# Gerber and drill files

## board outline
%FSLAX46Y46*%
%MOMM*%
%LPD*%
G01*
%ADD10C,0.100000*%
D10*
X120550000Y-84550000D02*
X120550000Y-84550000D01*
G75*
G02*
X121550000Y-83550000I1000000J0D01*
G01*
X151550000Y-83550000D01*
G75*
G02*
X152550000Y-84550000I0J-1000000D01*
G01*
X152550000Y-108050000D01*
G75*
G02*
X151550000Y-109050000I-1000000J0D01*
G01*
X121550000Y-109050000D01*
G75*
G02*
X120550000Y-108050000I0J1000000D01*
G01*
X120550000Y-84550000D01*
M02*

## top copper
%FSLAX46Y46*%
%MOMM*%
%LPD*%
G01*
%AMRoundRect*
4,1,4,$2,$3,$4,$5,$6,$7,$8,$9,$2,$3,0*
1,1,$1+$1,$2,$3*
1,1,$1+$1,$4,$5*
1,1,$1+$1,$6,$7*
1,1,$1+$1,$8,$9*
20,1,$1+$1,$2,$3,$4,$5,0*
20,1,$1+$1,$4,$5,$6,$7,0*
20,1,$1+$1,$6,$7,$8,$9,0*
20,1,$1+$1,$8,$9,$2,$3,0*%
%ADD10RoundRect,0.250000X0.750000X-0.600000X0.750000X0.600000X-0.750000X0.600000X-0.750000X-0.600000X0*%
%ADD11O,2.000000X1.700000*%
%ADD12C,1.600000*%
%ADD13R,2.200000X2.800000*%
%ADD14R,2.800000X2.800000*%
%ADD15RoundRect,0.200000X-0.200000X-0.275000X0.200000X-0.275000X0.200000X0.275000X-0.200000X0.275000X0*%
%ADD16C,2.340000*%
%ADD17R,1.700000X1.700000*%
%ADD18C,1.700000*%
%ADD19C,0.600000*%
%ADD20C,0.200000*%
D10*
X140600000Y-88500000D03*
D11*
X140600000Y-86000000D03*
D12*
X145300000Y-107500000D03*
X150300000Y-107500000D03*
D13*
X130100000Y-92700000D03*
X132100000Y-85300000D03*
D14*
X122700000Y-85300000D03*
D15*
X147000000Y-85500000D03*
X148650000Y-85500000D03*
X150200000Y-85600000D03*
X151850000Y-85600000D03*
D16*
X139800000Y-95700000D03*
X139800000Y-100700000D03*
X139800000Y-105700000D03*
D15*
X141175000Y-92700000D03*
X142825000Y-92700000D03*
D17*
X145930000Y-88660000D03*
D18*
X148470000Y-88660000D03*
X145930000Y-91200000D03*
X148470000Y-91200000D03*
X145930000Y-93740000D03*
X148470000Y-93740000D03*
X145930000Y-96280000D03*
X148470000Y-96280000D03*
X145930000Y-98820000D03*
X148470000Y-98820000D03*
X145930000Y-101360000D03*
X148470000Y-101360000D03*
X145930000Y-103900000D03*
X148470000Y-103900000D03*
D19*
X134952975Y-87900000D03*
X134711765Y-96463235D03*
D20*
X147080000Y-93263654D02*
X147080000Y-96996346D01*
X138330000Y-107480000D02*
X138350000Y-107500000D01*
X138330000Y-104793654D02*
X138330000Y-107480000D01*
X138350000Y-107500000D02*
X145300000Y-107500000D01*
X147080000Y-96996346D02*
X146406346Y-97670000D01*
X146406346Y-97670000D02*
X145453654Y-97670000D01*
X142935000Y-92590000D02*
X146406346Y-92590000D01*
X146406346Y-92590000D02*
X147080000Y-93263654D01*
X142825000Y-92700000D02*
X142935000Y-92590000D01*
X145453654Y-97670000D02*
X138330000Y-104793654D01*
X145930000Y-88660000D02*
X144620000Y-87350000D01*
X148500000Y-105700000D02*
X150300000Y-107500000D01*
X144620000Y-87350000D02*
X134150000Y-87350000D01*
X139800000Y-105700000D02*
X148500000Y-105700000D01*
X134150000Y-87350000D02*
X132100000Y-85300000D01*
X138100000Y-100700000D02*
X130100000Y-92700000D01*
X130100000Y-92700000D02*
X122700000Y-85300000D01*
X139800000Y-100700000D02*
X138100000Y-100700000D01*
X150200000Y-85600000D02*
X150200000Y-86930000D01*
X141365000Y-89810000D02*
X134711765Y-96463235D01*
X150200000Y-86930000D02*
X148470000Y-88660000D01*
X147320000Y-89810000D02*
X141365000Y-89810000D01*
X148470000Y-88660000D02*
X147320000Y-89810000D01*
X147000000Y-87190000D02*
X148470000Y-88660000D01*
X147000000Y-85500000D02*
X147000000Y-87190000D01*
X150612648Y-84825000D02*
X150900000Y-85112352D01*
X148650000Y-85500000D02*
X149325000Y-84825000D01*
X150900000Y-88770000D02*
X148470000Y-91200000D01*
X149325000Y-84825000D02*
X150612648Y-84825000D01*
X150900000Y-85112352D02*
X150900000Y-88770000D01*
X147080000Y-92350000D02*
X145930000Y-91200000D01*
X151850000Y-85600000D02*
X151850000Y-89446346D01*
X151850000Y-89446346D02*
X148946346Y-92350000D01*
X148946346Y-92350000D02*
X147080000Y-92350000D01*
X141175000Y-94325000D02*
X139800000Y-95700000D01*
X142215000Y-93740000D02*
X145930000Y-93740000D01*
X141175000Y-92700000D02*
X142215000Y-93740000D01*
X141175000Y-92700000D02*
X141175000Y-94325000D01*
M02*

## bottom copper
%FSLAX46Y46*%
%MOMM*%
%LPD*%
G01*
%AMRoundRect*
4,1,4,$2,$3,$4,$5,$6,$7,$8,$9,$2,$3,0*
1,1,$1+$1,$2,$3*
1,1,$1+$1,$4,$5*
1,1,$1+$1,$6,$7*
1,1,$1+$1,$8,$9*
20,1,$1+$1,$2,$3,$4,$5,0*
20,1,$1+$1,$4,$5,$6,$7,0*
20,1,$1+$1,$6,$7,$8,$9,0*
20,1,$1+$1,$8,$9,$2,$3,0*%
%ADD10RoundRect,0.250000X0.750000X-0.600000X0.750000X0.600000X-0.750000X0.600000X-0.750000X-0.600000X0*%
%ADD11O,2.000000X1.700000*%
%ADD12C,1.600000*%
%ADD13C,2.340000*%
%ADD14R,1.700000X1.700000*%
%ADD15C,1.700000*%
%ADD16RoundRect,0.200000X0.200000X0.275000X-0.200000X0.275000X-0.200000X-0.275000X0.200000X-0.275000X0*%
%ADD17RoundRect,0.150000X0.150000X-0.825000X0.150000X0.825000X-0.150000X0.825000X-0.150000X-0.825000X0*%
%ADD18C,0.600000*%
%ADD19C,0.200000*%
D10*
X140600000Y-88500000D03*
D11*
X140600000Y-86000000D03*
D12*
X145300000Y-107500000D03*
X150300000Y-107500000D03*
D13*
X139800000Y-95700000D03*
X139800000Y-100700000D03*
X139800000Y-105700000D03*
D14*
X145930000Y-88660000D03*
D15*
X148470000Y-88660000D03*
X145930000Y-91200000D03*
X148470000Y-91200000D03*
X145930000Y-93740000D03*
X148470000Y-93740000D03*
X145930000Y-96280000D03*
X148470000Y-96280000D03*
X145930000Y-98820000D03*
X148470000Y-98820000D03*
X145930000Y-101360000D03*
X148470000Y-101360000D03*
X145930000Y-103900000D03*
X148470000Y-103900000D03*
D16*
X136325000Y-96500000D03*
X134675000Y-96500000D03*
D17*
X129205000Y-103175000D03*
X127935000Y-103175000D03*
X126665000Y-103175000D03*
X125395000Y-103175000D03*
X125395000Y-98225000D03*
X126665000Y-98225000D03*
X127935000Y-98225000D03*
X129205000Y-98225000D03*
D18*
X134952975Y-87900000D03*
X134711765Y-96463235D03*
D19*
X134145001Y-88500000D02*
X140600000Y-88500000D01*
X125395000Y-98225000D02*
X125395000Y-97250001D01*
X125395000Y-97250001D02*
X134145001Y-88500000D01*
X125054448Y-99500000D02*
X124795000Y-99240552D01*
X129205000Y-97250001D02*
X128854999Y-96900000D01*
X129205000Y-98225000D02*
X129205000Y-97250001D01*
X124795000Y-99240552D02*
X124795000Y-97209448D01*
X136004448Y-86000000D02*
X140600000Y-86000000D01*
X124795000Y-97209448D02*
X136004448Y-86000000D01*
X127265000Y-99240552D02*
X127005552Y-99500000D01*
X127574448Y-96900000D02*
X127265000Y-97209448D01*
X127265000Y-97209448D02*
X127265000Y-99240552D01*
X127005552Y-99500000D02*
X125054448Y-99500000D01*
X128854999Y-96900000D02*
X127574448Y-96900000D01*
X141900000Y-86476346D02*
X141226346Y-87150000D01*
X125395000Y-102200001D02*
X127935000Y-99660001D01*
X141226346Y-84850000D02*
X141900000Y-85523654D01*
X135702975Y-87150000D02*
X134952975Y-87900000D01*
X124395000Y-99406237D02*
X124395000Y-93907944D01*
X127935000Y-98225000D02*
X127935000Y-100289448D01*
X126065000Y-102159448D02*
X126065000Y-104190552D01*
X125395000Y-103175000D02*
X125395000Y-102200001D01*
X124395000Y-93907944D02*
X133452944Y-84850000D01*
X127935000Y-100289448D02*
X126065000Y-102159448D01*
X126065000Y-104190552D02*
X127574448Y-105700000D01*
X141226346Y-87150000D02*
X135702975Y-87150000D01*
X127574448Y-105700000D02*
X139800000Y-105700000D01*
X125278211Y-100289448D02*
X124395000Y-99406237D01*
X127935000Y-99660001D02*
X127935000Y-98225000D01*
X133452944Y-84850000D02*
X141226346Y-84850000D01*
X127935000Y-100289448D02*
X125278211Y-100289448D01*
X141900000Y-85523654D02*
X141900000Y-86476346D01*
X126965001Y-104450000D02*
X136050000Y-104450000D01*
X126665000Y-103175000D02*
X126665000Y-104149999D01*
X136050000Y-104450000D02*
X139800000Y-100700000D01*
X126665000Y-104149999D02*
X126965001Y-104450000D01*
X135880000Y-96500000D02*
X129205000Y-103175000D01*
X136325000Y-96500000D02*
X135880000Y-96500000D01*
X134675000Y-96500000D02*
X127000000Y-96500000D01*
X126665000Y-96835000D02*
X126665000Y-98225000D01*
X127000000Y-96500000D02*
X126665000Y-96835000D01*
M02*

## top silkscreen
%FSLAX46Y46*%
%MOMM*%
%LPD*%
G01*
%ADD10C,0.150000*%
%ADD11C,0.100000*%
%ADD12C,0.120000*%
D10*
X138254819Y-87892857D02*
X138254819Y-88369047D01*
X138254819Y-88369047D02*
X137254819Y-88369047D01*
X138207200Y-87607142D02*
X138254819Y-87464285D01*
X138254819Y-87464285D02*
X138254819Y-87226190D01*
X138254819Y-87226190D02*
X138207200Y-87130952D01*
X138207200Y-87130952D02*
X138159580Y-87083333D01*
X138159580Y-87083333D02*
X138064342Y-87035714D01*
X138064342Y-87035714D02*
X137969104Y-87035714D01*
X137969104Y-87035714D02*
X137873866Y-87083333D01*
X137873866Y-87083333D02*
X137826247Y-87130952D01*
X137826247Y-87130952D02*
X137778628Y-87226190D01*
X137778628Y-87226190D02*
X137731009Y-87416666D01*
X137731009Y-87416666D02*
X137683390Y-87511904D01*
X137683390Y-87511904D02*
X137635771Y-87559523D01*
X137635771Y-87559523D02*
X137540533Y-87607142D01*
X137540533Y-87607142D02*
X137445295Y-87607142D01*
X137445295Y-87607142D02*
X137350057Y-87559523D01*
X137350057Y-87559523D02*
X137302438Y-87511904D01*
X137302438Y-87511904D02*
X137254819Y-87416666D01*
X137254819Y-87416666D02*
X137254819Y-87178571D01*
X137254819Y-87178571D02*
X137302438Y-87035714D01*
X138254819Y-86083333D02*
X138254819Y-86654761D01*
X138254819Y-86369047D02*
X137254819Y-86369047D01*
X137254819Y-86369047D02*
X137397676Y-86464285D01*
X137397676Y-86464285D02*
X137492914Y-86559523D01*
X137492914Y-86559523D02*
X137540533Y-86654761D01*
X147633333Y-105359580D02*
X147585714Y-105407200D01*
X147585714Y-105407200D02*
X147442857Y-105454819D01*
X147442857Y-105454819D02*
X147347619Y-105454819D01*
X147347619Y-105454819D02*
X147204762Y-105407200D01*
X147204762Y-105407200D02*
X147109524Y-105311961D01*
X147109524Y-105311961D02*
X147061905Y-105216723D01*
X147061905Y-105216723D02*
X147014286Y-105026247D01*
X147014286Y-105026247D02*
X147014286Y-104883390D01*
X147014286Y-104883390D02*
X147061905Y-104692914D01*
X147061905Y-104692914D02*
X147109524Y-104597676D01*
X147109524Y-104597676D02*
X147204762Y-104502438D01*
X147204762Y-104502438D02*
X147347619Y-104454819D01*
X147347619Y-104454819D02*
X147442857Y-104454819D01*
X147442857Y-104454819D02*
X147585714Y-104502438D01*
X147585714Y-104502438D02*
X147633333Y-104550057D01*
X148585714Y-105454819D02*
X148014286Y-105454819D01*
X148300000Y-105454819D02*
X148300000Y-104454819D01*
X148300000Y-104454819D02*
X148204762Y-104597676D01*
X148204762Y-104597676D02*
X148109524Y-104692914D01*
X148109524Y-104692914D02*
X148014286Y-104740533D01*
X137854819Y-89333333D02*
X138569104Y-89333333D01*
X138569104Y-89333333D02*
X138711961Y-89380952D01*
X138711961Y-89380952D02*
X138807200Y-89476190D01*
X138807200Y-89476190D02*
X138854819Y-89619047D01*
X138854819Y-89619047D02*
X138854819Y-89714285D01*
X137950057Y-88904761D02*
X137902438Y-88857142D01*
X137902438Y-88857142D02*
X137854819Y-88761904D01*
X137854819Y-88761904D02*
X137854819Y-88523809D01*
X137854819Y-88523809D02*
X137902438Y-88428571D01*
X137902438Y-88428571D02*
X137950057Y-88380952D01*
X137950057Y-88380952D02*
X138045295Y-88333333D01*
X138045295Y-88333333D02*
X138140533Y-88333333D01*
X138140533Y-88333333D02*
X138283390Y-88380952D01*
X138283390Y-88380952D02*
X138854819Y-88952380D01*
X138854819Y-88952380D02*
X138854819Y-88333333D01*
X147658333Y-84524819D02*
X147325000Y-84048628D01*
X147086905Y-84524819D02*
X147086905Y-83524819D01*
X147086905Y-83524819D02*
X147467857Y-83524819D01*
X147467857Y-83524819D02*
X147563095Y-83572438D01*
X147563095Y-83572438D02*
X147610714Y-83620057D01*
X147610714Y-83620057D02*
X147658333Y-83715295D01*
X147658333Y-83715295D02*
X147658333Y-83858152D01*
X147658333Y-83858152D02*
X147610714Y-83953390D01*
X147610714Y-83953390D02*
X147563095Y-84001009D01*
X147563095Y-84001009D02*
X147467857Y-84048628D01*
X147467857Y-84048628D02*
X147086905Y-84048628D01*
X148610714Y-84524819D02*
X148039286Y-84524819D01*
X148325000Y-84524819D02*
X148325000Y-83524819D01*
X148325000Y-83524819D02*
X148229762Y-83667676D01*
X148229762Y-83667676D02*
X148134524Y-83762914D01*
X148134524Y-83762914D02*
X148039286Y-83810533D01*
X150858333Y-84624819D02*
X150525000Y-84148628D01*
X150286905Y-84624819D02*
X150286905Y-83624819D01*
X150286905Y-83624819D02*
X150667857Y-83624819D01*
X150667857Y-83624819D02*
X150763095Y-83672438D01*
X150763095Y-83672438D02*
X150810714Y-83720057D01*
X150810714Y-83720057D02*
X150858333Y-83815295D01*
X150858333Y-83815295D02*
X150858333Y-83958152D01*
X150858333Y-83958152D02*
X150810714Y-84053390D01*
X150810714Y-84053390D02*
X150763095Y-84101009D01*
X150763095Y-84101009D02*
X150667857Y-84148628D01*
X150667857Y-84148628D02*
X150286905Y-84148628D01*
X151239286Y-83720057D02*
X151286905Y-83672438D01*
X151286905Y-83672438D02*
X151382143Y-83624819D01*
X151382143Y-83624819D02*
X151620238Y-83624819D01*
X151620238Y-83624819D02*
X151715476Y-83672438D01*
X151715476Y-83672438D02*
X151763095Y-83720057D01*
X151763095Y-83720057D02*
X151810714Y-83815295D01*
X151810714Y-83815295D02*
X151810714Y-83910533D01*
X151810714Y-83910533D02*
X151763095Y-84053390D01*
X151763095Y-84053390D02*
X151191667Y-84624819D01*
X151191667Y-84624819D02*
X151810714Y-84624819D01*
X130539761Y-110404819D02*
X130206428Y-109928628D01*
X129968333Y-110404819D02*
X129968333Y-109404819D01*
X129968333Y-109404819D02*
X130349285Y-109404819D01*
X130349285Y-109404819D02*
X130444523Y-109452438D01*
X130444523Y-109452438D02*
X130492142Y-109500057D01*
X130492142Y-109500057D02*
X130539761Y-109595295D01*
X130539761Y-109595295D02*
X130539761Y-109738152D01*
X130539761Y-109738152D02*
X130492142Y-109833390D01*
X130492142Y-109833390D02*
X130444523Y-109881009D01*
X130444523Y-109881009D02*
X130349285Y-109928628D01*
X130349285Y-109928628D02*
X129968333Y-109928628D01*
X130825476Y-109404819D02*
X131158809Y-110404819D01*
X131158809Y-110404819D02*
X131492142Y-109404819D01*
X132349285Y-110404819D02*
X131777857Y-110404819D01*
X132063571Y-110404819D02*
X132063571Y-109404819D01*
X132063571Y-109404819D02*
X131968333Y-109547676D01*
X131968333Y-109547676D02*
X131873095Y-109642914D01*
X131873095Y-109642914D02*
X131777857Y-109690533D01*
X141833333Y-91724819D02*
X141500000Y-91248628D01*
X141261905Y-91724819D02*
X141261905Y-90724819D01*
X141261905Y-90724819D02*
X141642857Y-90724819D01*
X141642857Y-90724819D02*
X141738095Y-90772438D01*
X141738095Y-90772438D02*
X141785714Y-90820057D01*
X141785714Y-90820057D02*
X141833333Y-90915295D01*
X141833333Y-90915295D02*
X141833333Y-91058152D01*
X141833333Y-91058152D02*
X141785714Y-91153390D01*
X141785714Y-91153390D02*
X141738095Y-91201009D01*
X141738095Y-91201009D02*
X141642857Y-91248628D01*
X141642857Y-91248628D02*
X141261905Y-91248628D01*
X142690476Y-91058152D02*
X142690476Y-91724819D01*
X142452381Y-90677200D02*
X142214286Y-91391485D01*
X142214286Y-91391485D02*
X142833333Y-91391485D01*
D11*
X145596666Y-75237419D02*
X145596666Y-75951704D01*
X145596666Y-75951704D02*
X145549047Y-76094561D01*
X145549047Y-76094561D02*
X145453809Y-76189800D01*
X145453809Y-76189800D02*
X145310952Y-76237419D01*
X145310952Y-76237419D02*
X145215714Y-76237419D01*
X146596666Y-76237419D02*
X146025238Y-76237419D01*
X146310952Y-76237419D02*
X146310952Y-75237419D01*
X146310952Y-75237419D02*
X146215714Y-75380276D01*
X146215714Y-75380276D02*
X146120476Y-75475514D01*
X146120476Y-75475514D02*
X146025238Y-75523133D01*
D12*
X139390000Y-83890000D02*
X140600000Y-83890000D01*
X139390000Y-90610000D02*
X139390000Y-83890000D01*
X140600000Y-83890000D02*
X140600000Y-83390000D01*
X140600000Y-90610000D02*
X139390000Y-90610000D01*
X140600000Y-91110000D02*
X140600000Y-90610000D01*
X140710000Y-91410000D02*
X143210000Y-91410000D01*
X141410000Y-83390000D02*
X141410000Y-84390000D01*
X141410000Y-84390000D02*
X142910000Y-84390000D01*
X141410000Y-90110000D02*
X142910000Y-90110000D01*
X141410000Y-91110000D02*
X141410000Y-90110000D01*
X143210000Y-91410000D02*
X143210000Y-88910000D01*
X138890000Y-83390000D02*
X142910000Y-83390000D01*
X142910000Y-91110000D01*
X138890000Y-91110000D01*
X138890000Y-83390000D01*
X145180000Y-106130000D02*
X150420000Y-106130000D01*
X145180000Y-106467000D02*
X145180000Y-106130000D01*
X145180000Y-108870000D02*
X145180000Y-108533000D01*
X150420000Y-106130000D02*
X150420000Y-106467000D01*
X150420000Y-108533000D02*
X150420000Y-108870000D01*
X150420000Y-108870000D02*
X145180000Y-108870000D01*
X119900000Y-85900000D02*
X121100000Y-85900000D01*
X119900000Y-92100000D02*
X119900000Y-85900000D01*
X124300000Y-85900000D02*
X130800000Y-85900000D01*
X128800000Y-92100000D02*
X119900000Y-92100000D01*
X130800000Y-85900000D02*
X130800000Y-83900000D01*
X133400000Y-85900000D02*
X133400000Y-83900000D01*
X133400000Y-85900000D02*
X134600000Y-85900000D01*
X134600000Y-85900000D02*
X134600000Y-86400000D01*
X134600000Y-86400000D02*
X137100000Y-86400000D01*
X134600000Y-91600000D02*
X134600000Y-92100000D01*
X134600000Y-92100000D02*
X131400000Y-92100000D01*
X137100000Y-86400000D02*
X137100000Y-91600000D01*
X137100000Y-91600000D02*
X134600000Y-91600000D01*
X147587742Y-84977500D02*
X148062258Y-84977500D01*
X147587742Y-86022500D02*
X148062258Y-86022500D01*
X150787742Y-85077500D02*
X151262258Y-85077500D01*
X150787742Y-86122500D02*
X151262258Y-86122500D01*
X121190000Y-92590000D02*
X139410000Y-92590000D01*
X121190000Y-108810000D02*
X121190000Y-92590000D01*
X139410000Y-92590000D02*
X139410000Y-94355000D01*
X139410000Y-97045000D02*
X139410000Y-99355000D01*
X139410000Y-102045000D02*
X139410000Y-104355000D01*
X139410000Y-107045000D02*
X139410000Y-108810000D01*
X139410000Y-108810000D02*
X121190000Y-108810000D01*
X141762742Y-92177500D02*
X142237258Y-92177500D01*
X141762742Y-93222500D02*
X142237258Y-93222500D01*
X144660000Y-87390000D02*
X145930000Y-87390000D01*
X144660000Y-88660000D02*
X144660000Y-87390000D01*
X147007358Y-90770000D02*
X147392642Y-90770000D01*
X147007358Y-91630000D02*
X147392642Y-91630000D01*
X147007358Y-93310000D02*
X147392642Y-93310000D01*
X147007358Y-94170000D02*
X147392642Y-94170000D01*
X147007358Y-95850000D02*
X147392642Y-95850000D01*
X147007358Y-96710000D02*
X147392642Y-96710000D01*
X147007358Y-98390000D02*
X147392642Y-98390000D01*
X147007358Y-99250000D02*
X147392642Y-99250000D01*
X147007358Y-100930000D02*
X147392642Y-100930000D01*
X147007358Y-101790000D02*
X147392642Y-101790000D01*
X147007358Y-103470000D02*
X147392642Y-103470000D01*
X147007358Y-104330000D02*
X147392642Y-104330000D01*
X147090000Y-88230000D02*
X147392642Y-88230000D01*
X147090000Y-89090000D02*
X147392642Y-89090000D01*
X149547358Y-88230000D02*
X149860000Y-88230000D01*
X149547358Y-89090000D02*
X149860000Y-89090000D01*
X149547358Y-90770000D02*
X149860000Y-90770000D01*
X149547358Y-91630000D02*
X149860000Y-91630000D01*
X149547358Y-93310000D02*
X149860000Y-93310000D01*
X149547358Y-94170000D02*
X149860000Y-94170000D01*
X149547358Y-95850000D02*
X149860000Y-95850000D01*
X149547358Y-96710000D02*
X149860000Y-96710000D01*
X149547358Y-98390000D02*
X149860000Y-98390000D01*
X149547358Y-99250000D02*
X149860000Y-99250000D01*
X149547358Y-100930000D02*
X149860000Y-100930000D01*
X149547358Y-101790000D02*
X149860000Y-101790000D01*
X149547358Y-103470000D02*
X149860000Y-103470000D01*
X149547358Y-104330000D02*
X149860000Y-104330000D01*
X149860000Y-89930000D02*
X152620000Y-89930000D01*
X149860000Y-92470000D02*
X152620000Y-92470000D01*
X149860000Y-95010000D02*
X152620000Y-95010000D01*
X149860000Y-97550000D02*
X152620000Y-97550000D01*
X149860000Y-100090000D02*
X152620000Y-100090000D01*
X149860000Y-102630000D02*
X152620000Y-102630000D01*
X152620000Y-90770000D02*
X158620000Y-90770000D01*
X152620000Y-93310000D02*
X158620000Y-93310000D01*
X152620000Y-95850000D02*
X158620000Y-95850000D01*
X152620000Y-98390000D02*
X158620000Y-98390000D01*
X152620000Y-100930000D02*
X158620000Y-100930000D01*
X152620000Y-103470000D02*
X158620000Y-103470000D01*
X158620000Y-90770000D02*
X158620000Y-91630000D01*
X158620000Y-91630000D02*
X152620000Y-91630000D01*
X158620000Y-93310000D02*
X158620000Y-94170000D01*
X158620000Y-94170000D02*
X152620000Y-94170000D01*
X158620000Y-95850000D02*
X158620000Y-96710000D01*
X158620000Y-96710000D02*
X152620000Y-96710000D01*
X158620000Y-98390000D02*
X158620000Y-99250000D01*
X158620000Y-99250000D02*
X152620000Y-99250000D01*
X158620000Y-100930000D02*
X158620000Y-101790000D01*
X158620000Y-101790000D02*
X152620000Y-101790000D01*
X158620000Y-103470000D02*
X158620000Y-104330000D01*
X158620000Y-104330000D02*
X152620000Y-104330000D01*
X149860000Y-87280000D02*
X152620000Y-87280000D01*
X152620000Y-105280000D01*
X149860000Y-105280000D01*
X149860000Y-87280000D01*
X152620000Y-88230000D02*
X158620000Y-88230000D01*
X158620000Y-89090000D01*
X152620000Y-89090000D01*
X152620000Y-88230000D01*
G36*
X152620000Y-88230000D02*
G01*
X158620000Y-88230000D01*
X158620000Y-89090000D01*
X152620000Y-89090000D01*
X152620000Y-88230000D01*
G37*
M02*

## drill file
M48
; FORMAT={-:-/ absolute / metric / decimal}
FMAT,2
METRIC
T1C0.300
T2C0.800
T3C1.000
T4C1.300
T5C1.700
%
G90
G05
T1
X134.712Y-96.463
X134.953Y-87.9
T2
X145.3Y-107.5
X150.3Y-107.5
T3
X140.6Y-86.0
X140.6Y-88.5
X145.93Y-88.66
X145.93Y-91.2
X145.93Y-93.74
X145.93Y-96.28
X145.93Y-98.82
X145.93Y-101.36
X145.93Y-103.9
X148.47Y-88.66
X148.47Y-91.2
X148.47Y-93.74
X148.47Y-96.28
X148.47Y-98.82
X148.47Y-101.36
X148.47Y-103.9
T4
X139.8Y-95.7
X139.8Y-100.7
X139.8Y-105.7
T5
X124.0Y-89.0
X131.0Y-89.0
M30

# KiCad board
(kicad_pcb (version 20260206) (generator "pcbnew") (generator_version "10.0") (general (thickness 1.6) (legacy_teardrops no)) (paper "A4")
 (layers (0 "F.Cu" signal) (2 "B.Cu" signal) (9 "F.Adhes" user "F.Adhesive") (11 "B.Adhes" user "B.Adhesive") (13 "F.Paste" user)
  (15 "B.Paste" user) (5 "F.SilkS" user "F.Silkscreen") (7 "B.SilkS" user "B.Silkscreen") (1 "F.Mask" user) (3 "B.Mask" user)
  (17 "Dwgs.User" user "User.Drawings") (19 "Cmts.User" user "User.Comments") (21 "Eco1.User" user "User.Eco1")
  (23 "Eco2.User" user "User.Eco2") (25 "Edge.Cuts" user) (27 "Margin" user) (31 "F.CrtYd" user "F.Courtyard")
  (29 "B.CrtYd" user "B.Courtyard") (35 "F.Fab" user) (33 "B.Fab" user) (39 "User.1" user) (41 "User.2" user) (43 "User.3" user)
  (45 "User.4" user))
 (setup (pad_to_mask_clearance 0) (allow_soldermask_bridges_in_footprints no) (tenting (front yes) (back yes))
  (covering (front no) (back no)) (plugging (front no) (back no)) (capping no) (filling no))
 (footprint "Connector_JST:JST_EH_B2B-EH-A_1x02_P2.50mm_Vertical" (layer "F.Cu") (at 140.6 88.5 90)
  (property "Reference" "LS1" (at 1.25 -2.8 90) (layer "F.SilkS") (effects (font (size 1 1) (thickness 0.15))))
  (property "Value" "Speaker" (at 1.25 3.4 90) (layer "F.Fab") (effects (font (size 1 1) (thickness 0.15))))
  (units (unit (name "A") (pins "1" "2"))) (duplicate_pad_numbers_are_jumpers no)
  (fp_line (start 4.61 -1.21) (end 4.61 0) (stroke (width 0.12) (type solid)) (layer "F.SilkS"))
  (fp_line (start -2.11 -1.21) (end 4.61 -1.21) (stroke (width 0.12) (type solid)) (layer "F.SilkS"))
  (fp_line (start 4.61 0) (end 5.11 0) (stroke (width 0.12) (type solid)) (layer "F.SilkS"))
  (fp_line (start -2.11 0) (end -2.11 -1.21) (stroke (width 0.12) (type solid)) (layer "F.SilkS"))
  (fp_line (start -2.61 0) (end -2.11 0) (stroke (width 0.12) (type solid)) (layer "F.SilkS"))
  (fp_line (start -2.91 0.11) (end -2.91 2.61) (stroke (width 0.12) (type solid)) (layer "F.SilkS"))
  (fp_line (start 5.11 0.81) (end 4.11 0.81) (stroke (width 0.12) (type solid)) (layer "F.SilkS"))
  (fp_line (start 4.11 0.81) (end 4.11 2.31) (stroke (width 0.12) (type solid)) (layer "F.SilkS"))
  (fp_line (start -1.61 0.81) (end -1.61 2.31) (stroke (width 0.12) (type solid)) (layer "F.SilkS"))
  (fp_line (start -2.61 0.81) (end -1.61 0.81) (stroke (width 0.12) (type solid)) (layer "F.SilkS"))
  (fp_line (start -2.91 2.61) (end -0.41 2.61) (stroke (width 0.12) (type solid)) (layer "F.SilkS"))
  (fp_rect (start -2.61 -1.71) (end 5.11 2.31) (stroke (width 0.12) (type solid)) (fill no) (layer "F.SilkS"))
  (pad "1" thru_hole roundrect (at 0 0 90) (size 1.7 2) (drill 1) (layers "*.Cu" "*.Mask") (remove_unused_layers no)
   (roundrect_rratio 0.147059) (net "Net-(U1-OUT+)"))
  (pad "2" thru_hole oval (at 2.5 0 90) (size 1.7 2) (drill 1) (layers "*.Cu" "*.Mask") (remove_unused_layers no) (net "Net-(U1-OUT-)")))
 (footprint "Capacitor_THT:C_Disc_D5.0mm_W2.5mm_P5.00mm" (layer "F.Cu") (at 145.3 107.5)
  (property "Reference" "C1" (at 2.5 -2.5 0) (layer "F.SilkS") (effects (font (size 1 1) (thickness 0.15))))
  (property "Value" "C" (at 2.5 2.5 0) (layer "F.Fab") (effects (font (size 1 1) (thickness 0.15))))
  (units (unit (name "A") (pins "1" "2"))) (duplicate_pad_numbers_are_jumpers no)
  (fp_line (start -0.12 -1.37) (end 5.12 -1.37) (stroke (width 0.12) (type solid)) (layer "F.SilkS"))
  (fp_line (start -0.12 -1.033) (end -0.12 -1.37) (stroke (width 0.12) (type solid)) (layer "F.SilkS"))
  (fp_line (start -0.12 1.37) (end -0.12 1.033) (stroke (width 0.12) (type solid)) (layer "F.SilkS"))
  (fp_line (start 5.12 -1.37) (end 5.12 -1.033) (stroke (width 0.12) (type solid)) (layer "F.SilkS"))
  (fp_line (start 5.12 1.033) (end 5.12 1.37) (stroke (width 0.12) (type solid)) (layer "F.SilkS"))
  (fp_line (start 5.12 1.37) (end -0.12 1.37) (stroke (width 0.12) (type solid)) (layer "F.SilkS"))
  (pad "1" thru_hole circle (at 0 0) (size 1.6 1.6) (drill 0.8) (layers "*.Cu" "*.Mask") (remove_unused_layers no) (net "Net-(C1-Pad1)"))
  (pad "2" thru_hole circle (at 5 0) (size 1.6 1.6) (drill 0.8) (layers "*.Cu" "*.Mask") (remove_unused_layers no) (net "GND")))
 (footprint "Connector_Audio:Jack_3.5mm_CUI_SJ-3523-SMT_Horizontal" (layer "F.Cu") (at 128.5 89 -90)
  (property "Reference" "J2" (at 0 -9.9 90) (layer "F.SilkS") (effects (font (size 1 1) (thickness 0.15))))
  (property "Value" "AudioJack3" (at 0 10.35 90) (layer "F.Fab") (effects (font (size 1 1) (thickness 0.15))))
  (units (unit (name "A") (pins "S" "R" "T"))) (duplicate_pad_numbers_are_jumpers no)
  (fp_line (start -3.1 8.6) (end -3.1 7.4) (stroke (width 0.12) (type solid)) (layer "F.SilkS"))
  (fp_line (start 3.1 8.6) (end -3.1 8.6) (stroke (width 0.12) (type solid)) (layer "F.SilkS"))
  (fp_line (start -3.1 4.2) (end -3.1 -2.3) (stroke (width 0.12) (type solid)) (layer "F.SilkS"))
  (fp_line (start 3.1 -0.3) (end 3.1 8.6) (stroke (width 0.12) (type solid)) (layer "F.SilkS"))
  (fp_line (start -3.1 -2.3) (end -5.1 -2.3) (stroke (width 0.12) (type solid)) (layer "F.SilkS"))
  (fp_line (start -3.1 -4.9) (end -5.1 -4.9) (stroke (width 0.12) (type solid)) (layer "F.SilkS"))
  (fp_line (start -3.1 -4.9) (end -3.1 -6.1) (stroke (width 0.12) (type solid)) (layer "F.SilkS"))
  (fp_line (start -3.1 -6.1) (end -2.6 -6.1) (stroke (width 0.12) (type solid)) (layer "F.SilkS"))
  (fp_line (start -2.6 -6.1) (end -2.6 -8.6) (stroke (width 0.12) (type solid)) (layer "F.SilkS"))
  (fp_line (start 2.6 -6.1) (end 3.1 -6.1) (stroke (width 0.12) (type solid)) (layer "F.SilkS"))
  (fp_line (start 3.1 -6.1) (end 3.1 -2.9) (stroke (width 0.12) (type solid)) (layer "F.SilkS"))
  (fp_line (start -2.6 -8.6) (end 2.6 -8.6) (stroke (width 0.12) (type solid)) (layer "F.SilkS"))
  (fp_line (start 2.6 -8.6) (end 2.6 -6.1) (stroke (width 0.12) (type solid)) (layer "F.SilkS"))
  (pad "" np_thru_hole circle (at 0 -2.5 270) (size 1.7 1.7) (drill 1.7) (layers "*.Cu" "*.Mask"))
  (pad "" np_thru_hole circle (at 0 4.5 270) (size 1.7 1.7) (drill 1.7) (layers "*.Cu" "*.Mask"))
  (pad "R" smd rect (at 3.7 -1.6 270) (size 2.8 2.2) (layers "F.Cu" "F.Mask" "F.Paste") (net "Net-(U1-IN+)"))
  (pad "S" smd rect (at -3.7 -3.6 270) (size 2.8 2.2) (layers "F.Cu" "F.Mask" "F.Paste") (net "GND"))
  (pad "T" smd rect (at -3.7 5.8 270) (size 2.8 2.8) (layers "F.Cu" "F.Mask" "F.Paste") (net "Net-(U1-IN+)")))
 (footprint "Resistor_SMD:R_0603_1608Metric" (layer "F.Cu") (at 147.825 85.5)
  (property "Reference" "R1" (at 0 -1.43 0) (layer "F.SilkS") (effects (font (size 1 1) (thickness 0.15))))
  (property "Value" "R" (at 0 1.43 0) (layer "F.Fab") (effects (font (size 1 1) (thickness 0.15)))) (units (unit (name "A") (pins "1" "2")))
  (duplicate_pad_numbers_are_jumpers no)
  (fp_line (start -0.237258 -0.5225) (end 0.237258 -0.5225) (stroke (width 0.12) (type solid)) (layer "F.SilkS"))
  (fp_line (start -0.237258 0.5225) (end 0.237258 0.5225) (stroke (width 0.12) (type solid)) (layer "F.SilkS"))
  (pad "1" smd roundrect (at -0.825 0) (size 0.8 0.95) (layers "F.Cu" "F.Mask" "F.Paste") (roundrect_rratio 0.25) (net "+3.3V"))
  (pad "2" smd roundrect (at 0.825 0) (size 0.8 0.95) (layers "F.Cu" "F.Mask" "F.Paste") (roundrect_rratio 0.25) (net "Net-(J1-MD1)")))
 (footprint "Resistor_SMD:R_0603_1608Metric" (layer "F.Cu") (at 151.025 85.6)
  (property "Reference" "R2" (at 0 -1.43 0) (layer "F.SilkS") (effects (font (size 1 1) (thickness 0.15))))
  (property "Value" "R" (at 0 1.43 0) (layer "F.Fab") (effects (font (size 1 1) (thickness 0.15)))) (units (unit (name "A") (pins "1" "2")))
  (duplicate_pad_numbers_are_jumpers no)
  (fp_line (start -0.237258 -0.5225) (end 0.237258 -0.5225) (stroke (width 0.12) (type solid)) (layer "F.SilkS"))
  (fp_line (start -0.237258 0.5225) (end 0.237258 0.5225) (stroke (width 0.12) (type solid)) (layer "F.SilkS"))
  (pad "1" smd roundrect (at -0.825 0) (size 0.8 0.95) (layers "F.Cu" "F.Mask" "F.Paste") (roundrect_rratio 0.25) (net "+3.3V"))
  (pad "2" smd roundrect (at 0.825 0) (size 0.8 0.95) (layers "F.Cu" "F.Mask" "F.Paste") (roundrect_rratio 0.25) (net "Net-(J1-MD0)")))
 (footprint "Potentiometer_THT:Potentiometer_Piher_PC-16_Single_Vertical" (layer "F.Cu") (at 139.8 95.7 180)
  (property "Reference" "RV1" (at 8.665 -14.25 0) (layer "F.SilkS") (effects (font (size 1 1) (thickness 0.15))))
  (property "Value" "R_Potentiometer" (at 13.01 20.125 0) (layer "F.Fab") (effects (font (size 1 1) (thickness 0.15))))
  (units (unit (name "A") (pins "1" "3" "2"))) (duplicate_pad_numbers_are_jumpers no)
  (fp_line (start 18.61 3.11) (end 0.39 3.11) (stroke (width 0.12) (type solid)) (layer "F.SilkS"))
  (fp_line (start 18.61 -13.11) (end 18.61 3.11) (stroke (width 0.12) (type solid)) (layer "F.SilkS"))
  (fp_line (start 0.39 3.11) (end 0.39 1.345) (stroke (width 0.12) (type solid)) (layer "F.SilkS"))
  (fp_line (start 0.39 -1.345) (end 0.39 -3.655) (stroke (width 0.12) (type solid)) (layer "F.SilkS"))
  (fp_line (start 0.39 -6.345) (end 0.39 -8.655) (stroke (width 0.12) (type solid)) (layer "F.SilkS"))
  (fp_line (start 0.39 -11.345) (end 0.39 -13.11) (stroke (width 0.12) (type solid)) (layer "F.SilkS"))
  (fp_line (start 0.39 -13.11) (end 18.61 -13.11) (stroke (width 0.12) (type solid)) (layer "F.SilkS"))
  (pad "1" thru_hole circle (at 0 0 180) (size 2.34 2.34) (drill 1.3) (layers "*.Cu" "*.Mask") (remove_unused_layers no)
   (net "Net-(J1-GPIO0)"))
  (pad "2" thru_hole circle (at 0 -5 180) (size 2.34 2.34) (drill 1.3) (layers "*.Cu" "*.Mask") (remove_unused_layers no)
   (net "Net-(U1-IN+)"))
  (pad "3" thru_hole circle (at 0 -10 180) (size 2.34 2.34) (drill 1.3) (layers "*.Cu" "*.Mask") (remove_unused_layers no) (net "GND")))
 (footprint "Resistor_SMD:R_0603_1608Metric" (layer "F.Cu") (at 142 92.7)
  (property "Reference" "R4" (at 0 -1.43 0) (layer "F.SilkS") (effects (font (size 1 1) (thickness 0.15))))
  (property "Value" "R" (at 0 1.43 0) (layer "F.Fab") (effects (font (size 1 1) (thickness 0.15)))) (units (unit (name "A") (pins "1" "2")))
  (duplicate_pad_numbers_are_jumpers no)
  (fp_line (start -0.237258 -0.5225) (end 0.237258 -0.5225) (stroke (width 0.12) (type solid)) (layer "F.SilkS"))
  (fp_line (start -0.237258 0.5225) (end 0.237258 0.5225) (stroke (width 0.12) (type solid)) (layer "F.SilkS"))
  (pad "1" smd roundrect (at -0.825 0) (size 0.8 0.95) (layers "F.Cu" "F.Mask" "F.Paste") (roundrect_rratio 0.25) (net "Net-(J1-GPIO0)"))
  (pad "2" smd roundrect (at 0.825 0) (size 0.8 0.95) (layers "F.Cu" "F.Mask" "F.Paste") (roundrect_rratio 0.25) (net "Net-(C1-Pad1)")))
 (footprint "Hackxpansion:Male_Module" (layer "F.Cu") (at 145.93 88.66)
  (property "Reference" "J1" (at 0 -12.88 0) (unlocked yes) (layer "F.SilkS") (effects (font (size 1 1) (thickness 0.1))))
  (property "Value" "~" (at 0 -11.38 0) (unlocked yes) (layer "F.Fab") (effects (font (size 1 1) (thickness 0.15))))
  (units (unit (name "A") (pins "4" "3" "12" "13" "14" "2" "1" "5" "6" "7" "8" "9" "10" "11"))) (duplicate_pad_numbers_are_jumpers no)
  (fp_line (start -1.27 -1.27) (end 0 -1.27) (stroke (width 0.12) (type solid)) (layer "F.SilkS"))
  (fp_line (start -1.27 0) (end -1.27 -1.27) (stroke (width 0.12) (type solid)) (layer "F.SilkS"))
  (fp_line (start 1.077358 2.11) (end 1.462642 2.11) (stroke (width 0.12) (type solid)) (layer "F.SilkS"))
  (fp_line (start 1.077358 2.97) (end 1.462642 2.97) (stroke (width 0.12) (type solid)) (layer "F.SilkS"))
  (fp_line (start 1.077358 4.65) (end 1.462642 4.65) (stroke (width 0.12) (type solid)) (layer "F.SilkS"))
  (fp_line (start 1.077358 5.51) (end 1.462642 5.51) (stroke (width 0.12) (type solid)) (layer "F.SilkS"))
  (fp_line (start 1.077358 7.19) (end 1.462642 7.19) (stroke (width 0.12) (type solid)) (layer "F.SilkS"))
  (fp_line (start 1.077358 8.05) (end 1.462642 8.05) (stroke (width 0.12) (type solid)) (layer "F.SilkS"))
  (fp_line (start 1.077358 9.73) (end 1.462642 9.73) (stroke (width 0.12) (type solid)) (layer "F.SilkS"))
  (fp_line (start 1.077358 10.59) (end 1.462642 10.59) (stroke (width 0.12) (type solid)) (layer "F.SilkS"))
  (fp_line (start 1.077358 12.27) (end 1.462642 12.27) (stroke (width 0.12) (type solid)) (layer "F.SilkS"))
  (fp_line (start 1.077358 13.13) (end 1.462642 13.13) (stroke (width 0.12) (type solid)) (layer "F.SilkS"))
  (fp_line (start 1.077358 14.81) (end 1.462642 14.81) (stroke (width 0.12) (type solid)) (layer "F.SilkS"))
  (fp_line (start 1.077358 15.67) (end 1.462642 15.67) (stroke (width 0.12) (type solid)) (layer "F.SilkS"))
  (fp_line (start 1.16 -0.43) (end 1.462642 -0.43) (stroke (width 0.12) (type solid)) (layer "F.SilkS"))
  (fp_line (start 1.16 0.43) (end 1.462642 0.43) (stroke (width 0.12) (type solid)) (layer "F.SilkS"))
  (fp_line (start 3.617358 -0.43) (end 3.93 -0.43) (stroke (width 0.12) (type solid)) (layer "F.SilkS"))
  (fp_line (start 3.617358 0.43) (end 3.93 0.43) (stroke (width 0.12) (type solid)) (layer "F.SilkS"))
  (fp_line (start 3.617358 2.11) (end 3.93 2.11) (stroke (width 0.12) (type solid)) (layer "F.SilkS"))
  (fp_line (start 3.617358 2.97) (end 3.93 2.97) (stroke (width 0.12) (type solid)) (layer "F.SilkS"))
  (fp_line (start 3.617358 4.65) (end 3.93 4.65) (stroke (width 0.12) (type solid)) (layer "F.SilkS"))
  (fp_line (start 3.617358 5.51) (end 3.93 5.51) (stroke (width 0.12) (type solid)) (layer "F.SilkS"))
  (fp_line (start 3.617358 7.19) (end 3.93 7.19) (stroke (width 0.12) (type solid)) (layer "F.SilkS"))
  (fp_line (start 3.617358 8.05) (end 3.93 8.05) (stroke (width 0.12) (type solid)) (layer "F.SilkS"))
  (fp_line (start 3.617358 9.73) (end 3.93 9.73) (stroke (width 0.12) (type solid)) (layer "F.SilkS"))
  (fp_line (start 3.617358 10.59) (end 3.93 10.59) (stroke (width 0.12) (type solid)) (layer "F.SilkS"))
  (fp_line (start 3.617358 12.27) (end 3.93 12.27) (stroke (width 0.12) (type solid)) (layer "F.SilkS"))
  (fp_line (start 3.617358 13.13) (end 3.93 13.13) (stroke (width 0.12) (type solid)) (layer "F.SilkS"))
  (fp_line (start 3.617358 14.81) (end 3.93 14.81) (stroke (width 0.12) (type solid)) (layer "F.SilkS"))
  (fp_line (start 3.617358 15.67) (end 3.93 15.67) (stroke (width 0.12) (type solid)) (layer "F.SilkS"))
  (fp_line (start 3.93 1.27) (end 6.69 1.27) (stroke (width 0.12) (type solid)) (layer "F.SilkS"))
  (fp_line (start 3.93 3.81) (end 6.69 3.81) (stroke (width 0.12) (type solid)) (layer "F.SilkS"))
  (fp_line (start 3.93 6.35) (end 6.69 6.35) (stroke (width 0.12) (type solid)) (layer "F.SilkS"))
  (fp_line (start 3.93 8.89) (end 6.69 8.89) (stroke (width 0.12) (type solid)) (layer "F.SilkS"))
  (fp_line (start 3.93 11.43) (end 6.69 11.43) (stroke (width 0.12) (type solid)) (layer "F.SilkS"))
  (fp_line (start 3.93 13.97) (end 6.69 13.97) (stroke (width 0.12) (type solid)) (layer "F.SilkS"))
  (fp_line (start 6.69 2.11) (end 12.69 2.11) (stroke (width 0.12) (type solid)) (layer "F.SilkS"))
  (fp_line (start 6.69 4.65) (end 12.69 4.65) (stroke (width 0.12) (type solid)) (layer "F.SilkS"))
  (fp_line (start 6.69 7.19) (end 12.69 7.19) (stroke (width 0.12) (type solid)) (layer "F.SilkS"))
  (fp_line (start 6.69 9.73) (end 12.69 9.73) (stroke (width 0.12) (type solid)) (layer "F.SilkS"))
  (fp_line (start 6.69 12.27) (end 12.69 12.27) (stroke (width 0.12) (type solid)) (layer "F.SilkS"))
  (fp_line (start 6.69 14.81) (end 12.69 14.81) (stroke (width 0.12) (type solid)) (layer "F.SilkS"))
  (fp_line (start 12.69 2.11) (end 12.69 2.97) (stroke (width 0.12) (type solid)) (layer "F.SilkS"))
  (fp_line (start 12.69 2.97) (end 6.69 2.97) (stroke (width 0.12) (type solid)) (layer "F.SilkS"))
  (fp_line (start 12.69 4.65) (end 12.69 5.51) (stroke (width 0.12) (type solid)) (layer "F.SilkS"))
  (fp_line (start 12.69 5.51) (end 6.69 5.51) (stroke (width 0.12) (type solid)) (layer "F.SilkS"))
  (fp_line (start 12.69 7.19) (end 12.69 8.05) (stroke (width 0.12) (type solid)) (layer "F.SilkS"))
  (fp_line (start 12.69 8.05) (end 6.69 8.05) (stroke (width 0.12) (type solid)) (layer "F.SilkS"))
  (fp_line (start 12.69 9.73) (end 12.69 10.59) (stroke (width 0.12) (type solid)) (layer "F.SilkS"))
  (fp_line (start 12.69 10.59) (end 6.69 10.59) (stroke (width 0.12) (type solid)) (layer "F.SilkS"))
  (fp_line (start 12.69 12.27) (end 12.69 13.13) (stroke (width 0.12) (type solid)) (layer "F.SilkS"))
  (fp_line (start 12.69 13.13) (end 6.69 13.13) (stroke (width 0.12) (type solid)) (layer "F.SilkS"))
  (fp_line (start 12.69 14.81) (end 12.69 15.67) (stroke (width 0.12) (type solid)) (layer "F.SilkS"))
  (fp_line (start 12.69 15.67) (end 6.69 15.67) (stroke (width 0.12) (type solid)) (layer "F.SilkS"))
  (fp_rect (start 3.93 -1.38) (end 6.69 16.62) (stroke (width 0.12) (type solid)) (fill no) (layer "F.SilkS"))
  (fp_rect (start 6.69 -0.43) (end 12.69 0.43) (stroke (width 0.12) (type solid)) (fill yes) (layer "F.SilkS"))
  (fp_rect (start -25.38 -5.11) (end 6.62 20.39) (radius 1) (stroke (width 0.1) (type solid)) (fill no) (layer "Edge.Cuts"))
  (pad "1" thru_hole rect (at 0 0) (size 1.7 1.7) (drill 1) (layers "*.Cu" "*.Mask") (remove_unused_layers no) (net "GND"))
  (pad "2" thru_hole circle (at 2.54 0) (size 1.7 1.7) (drill 1) (layers "*.Cu" "*.Mask") (remove_unused_layers no) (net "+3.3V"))
  (pad "3" thru_hole circle (at 0 2.54) (size 1.7 1.7) (drill 1) (layers "*.Cu" "*.Mask") (remove_unused_layers no) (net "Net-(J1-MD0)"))
  (pad "4" thru_hole circle (at 2.54 2.54) (size 1.7 1.7) (drill 1) (layers "*.Cu" "*.Mask") (remove_unused_layers no) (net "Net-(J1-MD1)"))
  (pad "5" thru_hole circle (at 0 5.08) (size 1.7 1.7) (drill 1) (layers "*.Cu" "*.Mask") (remove_unused_layers no) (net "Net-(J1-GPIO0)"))
  (pad "6" thru_hole circle (at 2.54 5.08) (size 1.7 1.7) (drill 1) (layers "*.Cu" "*.Mask") (remove_unused_layers no)
   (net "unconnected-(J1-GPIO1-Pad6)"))
  (pad "7" thru_hole circle (at 0 7.62) (size 1.7 1.7) (drill 1) (layers "*.Cu" "*.Mask") (remove_unused_layers no)
   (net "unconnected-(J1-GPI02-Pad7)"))
  (pad "8" thru_hole circle (at 2.54 7.62) (size 1.7 1.7) (drill 1) (layers "*.Cu" "*.Mask") (remove_unused_layers no)
   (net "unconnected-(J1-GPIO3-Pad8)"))
  (pad "9" thru_hole circle (at 0 10.16) (size 1.7 1.7) (drill 1) (layers "*.Cu" "*.Mask") (remove_unused_layers no)
   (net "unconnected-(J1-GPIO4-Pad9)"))
  (pad "10" thru_hole circle (at 2.54 10.16) (size 1.7 1.7) (drill 1) (layers "*.Cu" "*.Mask") (remove_unused_layers no)
   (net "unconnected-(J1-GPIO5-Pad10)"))
  (pad "11" thru_hole circle (at 0 12.7) (size 1.7 1.7) (drill 1) (layers "*.Cu" "*.Mask") (remove_unused_layers no)
   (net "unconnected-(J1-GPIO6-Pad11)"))
  (pad "12" thru_hole circle (at 2.54 12.7) (size 1.7 1.7) (drill 1) (layers "*.Cu" "*.Mask") (remove_unused_layers no)
   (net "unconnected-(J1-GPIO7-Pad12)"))
  (pad "13" thru_hole circle (at 0 15.24) (size 1.7 1.7) (drill 1) (layers "*.Cu" "*.Mask") (remove_unused_layers no)
   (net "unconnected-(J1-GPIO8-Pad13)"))
  (pad "14" thru_hole circle (at 2.54 15.24) (size 1.7 1.7) (drill 1) (layers "*.Cu" "*.Mask") (remove_unused_layers no)
   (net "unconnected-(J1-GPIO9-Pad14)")))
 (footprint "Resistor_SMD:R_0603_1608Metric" (layer "B.Cu") (at 135.5 96.5 180)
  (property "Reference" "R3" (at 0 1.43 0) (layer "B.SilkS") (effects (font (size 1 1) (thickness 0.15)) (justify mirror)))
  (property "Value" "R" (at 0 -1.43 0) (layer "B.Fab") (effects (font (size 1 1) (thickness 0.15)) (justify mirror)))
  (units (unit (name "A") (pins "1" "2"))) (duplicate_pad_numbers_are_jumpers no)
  (pad "1" smd roundrect (at -0.825 0 180) (size 0.8 0.95) (layers "B.Cu" "B.Mask" "B.Paste") (roundrect_rratio 0.25) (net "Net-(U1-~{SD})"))
  (pad "2" smd roundrect (at 0.825 0 180) (size 0.8 0.95) (layers "B.Cu" "B.Mask" "B.Paste") (roundrect_rratio 0.25) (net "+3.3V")))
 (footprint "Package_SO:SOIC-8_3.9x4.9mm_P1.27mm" (layer "B.Cu") (at 127.3 100.7 90)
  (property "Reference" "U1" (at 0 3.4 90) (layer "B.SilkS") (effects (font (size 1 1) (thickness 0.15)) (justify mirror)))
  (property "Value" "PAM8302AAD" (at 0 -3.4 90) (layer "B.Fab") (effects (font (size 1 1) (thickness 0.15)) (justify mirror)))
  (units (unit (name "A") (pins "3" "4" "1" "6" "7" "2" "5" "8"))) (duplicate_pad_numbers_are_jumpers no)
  (pad "1" smd roundrect (at -2.475 1.905 90) (size 1.95 0.6) (layers "B.Cu" "B.Mask" "B.Paste") (roundrect_rratio 0.25)
   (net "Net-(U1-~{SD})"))
  (pad "2" smd roundrect (at -2.475 0.635 90) (size 1.95 0.6) (layers "B.Cu" "B.Mask" "B.Paste") (roundrect_rratio 0.25)
   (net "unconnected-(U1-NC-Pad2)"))
  (pad "3" smd roundrect (at -2.475 -0.635 90) (size 1.95 0.6) (layers "B.Cu" "B.Mask" "B.Paste") (roundrect_rratio 0.25)
   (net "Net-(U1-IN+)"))
  (pad "4" smd roundrect (at -2.475 -1.905 90) (size 1.95 0.6) (layers "B.Cu" "B.Mask" "B.Paste") (roundrect_rratio 0.25) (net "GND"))
  (pad "5" smd roundrect (at 2.475 -1.905 90) (size 1.95 0.6) (layers "B.Cu" "B.Mask" "B.Paste") (roundrect_rratio 0.25)
   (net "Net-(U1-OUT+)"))
  (pad "6" smd roundrect (at 2.475 -0.635 90) (size 1.95 0.6) (layers "B.Cu" "B.Mask" "B.Paste") (roundrect_rratio 0.25) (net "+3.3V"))
  (pad "7" smd roundrect (at 2.475 0.635 90) (size 1.95 0.6) (layers "B.Cu" "B.Mask" "B.Paste") (roundrect_rratio 0.25) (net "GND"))
  (pad "8" smd roundrect (at 2.475 1.905 90) (size 1.95 0.6) (layers "B.Cu" "B.Mask" "B.Paste") (roundrect_rratio 0.25)
   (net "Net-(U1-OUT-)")))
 (segment (start 134.145001 88.5) (end 140.6 88.5) (width 0.2) (layer "B.Cu") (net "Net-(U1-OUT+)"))
 (segment (start 125.395 98.225) (end 125.395 97.250001) (width 0.2) (layer "B.Cu") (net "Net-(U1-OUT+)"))
 (segment (start 125.395 97.250001) (end 134.145001 88.5) (width 0.2) (layer "B.Cu") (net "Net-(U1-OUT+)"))
 (segment (start 125.054448 99.5) (end 124.795 99.240552) (width 0.2) (layer "B.Cu") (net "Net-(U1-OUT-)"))
 (segment (start 129.205 97.250001) (end 128.854999 96.9) (width 0.2) (layer "B.Cu") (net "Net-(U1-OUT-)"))
 (segment (start 129.205 98.225) (end 129.205 97.250001) (width 0.2) (layer "B.Cu") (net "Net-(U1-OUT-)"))
 (segment (start 124.795 99.240552) (end 124.795 97.209448) (width 0.2) (layer "B.Cu") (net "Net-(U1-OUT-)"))
 (segment (start 136.004448 86) (end 140.6 86) (width 0.2) (layer "B.Cu") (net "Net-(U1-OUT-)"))
 (segment (start 124.795 97.209448) (end 136.004448 86) (width 0.2) (layer "B.Cu") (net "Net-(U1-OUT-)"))
 (segment (start 127.265 99.240552) (end 127.005552 99.5) (width 0.2) (layer "B.Cu") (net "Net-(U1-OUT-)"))
 (segment (start 127.574448 96.9) (end 127.265 97.209448) (width 0.2) (layer "B.Cu") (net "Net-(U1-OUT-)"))
 (segment (start 127.265 97.209448) (end 127.265 99.240552) (width 0.2) (layer "B.Cu") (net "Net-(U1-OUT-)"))
 (segment (start 127.005552 99.5) (end 125.054448 99.5) (width 0.2) (layer "B.Cu") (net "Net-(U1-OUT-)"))
 (segment (start 128.854999 96.9) (end 127.574448 96.9) (width 0.2) (layer "B.Cu") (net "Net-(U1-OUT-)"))
 (segment (start 147.08 93.263654) (end 147.08 96.996346) (width 0.2) (layer "F.Cu") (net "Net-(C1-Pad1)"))
 (segment (start 138.33 107.48) (end 138.35 107.5) (width 0.2) (layer "F.Cu") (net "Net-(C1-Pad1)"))
 (segment (start 138.33 104.793654) (end 138.33 107.48) (width 0.2) (layer "F.Cu") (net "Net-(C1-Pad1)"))
 (segment (start 138.35 107.5) (end 145.3 107.5) (width 0.2) (layer "F.Cu") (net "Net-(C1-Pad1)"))
 (segment (start 147.08 96.996346) (end 146.406346 97.67) (width 0.2) (layer "F.Cu") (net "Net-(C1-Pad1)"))
 (segment (start 146.406346 97.67) (end 145.453654 97.67) (width 0.2) (layer "F.Cu") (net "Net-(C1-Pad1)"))
 (segment (start 142.935 92.59) (end 146.406346 92.59) (width 0.2) (layer "F.Cu") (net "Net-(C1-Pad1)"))
 (segment (start 146.406346 92.59) (end 147.08 93.263654) (width 0.2) (layer "F.Cu") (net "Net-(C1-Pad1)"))
 (segment (start 142.825 92.7) (end 142.935 92.59) (width 0.2) (layer "F.Cu") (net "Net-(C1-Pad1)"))
 (segment (start 145.453654 97.67) (end 138.33 104.793654) (width 0.2) (layer "F.Cu") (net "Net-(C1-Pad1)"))
 (segment (start 145.93 88.66) (end 144.62 87.35) (width 0.2) (layer "F.Cu") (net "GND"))
 (segment (start 148.5 105.7) (end 150.3 107.5) (width 0.2) (layer "F.Cu") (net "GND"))
 (segment (start 144.62 87.35) (end 134.15 87.35) (width 0.2) (layer "F.Cu") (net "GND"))
 (segment (start 139.8 105.7) (end 148.5 105.7) (width 0.2) (layer "F.Cu") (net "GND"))
 (segment (start 134.15 87.35) (end 132.1 85.3) (width 0.2) (layer "F.Cu") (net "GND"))
 (via (at 134.952975 87.9) (size 0.6) (drill 0.3) (layers "F.Cu" "B.Cu") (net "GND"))
 (segment (start 141.9 86.476346) (end 141.226346 87.15) (width 0.2) (layer "B.Cu") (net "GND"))
 (segment (start 125.395 102.200001) (end 127.935 99.660001) (width 0.2) (layer "B.Cu") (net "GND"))
 (segment (start 141.226346 84.85) (end 141.9 85.523654) (width 0.2) (layer "B.Cu") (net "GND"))
 (segment (start 135.702975 87.15) (end 134.952975 87.9) (width 0.2) (layer "B.Cu") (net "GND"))
 (segment (start 124.395 99.406237) (end 124.395 93.907944) (width 0.2) (layer "B.Cu") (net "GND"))
 (segment (start 127.935 98.225) (end 127.935 100.289448) (width 0.2) (layer "B.Cu") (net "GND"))
 (segment (start 126.065 102.159448) (end 126.065 104.190552) (width 0.2) (layer "B.Cu") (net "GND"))
 (segment (start 125.395 103.175) (end 125.395 102.200001) (width 0.2) (layer "B.Cu") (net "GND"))
 (segment (start 124.395 93.907944) (end 133.452944 84.85) (width 0.2) (layer "B.Cu") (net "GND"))
 (segment (start 127.935 100.289448) (end 126.065 102.159448) (width 0.2) (layer "B.Cu") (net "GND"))
 (segment (start 126.065 104.190552) (end 127.574448 105.7) (width 0.2) (layer "B.Cu") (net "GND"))
 (segment (start 141.226346 87.15) (end 135.702975 87.15) (width 0.2) (layer "B.Cu") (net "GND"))
 (segment (start 127.574448 105.7) (end 139.8 105.7) (width 0.2) (layer "B.Cu") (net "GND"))
 (segment (start 125.278211 100.289448) (end 124.395 99.406237) (width 0.2) (layer "B.Cu") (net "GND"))
 (segment (start 127.935 99.660001) (end 127.935 98.225) (width 0.2) (layer "B.Cu") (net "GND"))
 (segment (start 133.452944 84.85) (end 141.226346 84.85) (width 0.2) (layer "B.Cu") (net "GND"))
 (segment (start 127.935 100.289448) (end 125.278211 100.289448) (width 0.2) (layer "B.Cu") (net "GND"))
 (segment (start 141.9 85.523654) (end 141.9 86.476346) (width 0.2) (layer "B.Cu") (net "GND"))
 (segment (start 138.1 100.7) (end 130.1 92.7) (width 0.2) (layer "F.Cu") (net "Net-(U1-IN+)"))
 (segment (start 130.1 92.7) (end 122.7 85.3) (width 0.2) (layer "F.Cu") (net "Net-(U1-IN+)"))
 (segment (start 139.8 100.7) (end 138.1 100.7) (width 0.2) (layer "F.Cu") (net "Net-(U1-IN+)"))
 (segment (start 126.965001 104.45) (end 136.05 104.45) (width 0.2) (layer "B.Cu") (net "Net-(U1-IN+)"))
 (segment (start 126.665 103.175) (end 126.665 104.149999) (width 0.2) (layer "B.Cu") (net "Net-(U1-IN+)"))
 (segment (start 136.05 104.45) (end 139.8 100.7) (width 0.2) (layer "B.Cu") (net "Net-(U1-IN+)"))
 (segment (start 126.665 104.149999) (end 126.965001 104.45) (width 0.2) (layer "B.Cu") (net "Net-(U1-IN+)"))
 (segment (start 135.88 96.5) (end 129.205 103.175) (width 0.2) (layer "B.Cu") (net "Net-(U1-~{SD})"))
 (segment (start 136.325 96.5) (end 135.88 96.5) (width 0.2) (layer "B.Cu") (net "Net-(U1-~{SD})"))
 (segment (start 150.2 85.6) (end 150.2 86.93) (width 0.2) (layer "F.Cu") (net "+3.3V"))
 (segment (start 141.365 89.81) (end 134.711765 96.463235) (width 0.2) (layer "F.Cu") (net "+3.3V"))
 (segment (start 150.2 86.93) (end 148.47 88.66) (width 0.2) (layer "F.Cu") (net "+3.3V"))
 (segment (start 147.32 89.81) (end 141.365 89.81) (width 0.2) (layer "F.Cu") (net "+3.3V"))
 (segment (start 148.47 88.66) (end 147.32 89.81) (width 0.2) (layer "F.Cu") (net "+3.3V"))
 (segment (start 147 87.19) (end 148.47 88.66) (width 0.2) (layer "F.Cu") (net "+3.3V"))
 (segment (start 147 85.5) (end 147 87.19) (width 0.2) (layer "F.Cu") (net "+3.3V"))
 (via (at 134.711765 96.463235) (size 0.6) (drill 0.3) (layers "F.Cu" "B.Cu") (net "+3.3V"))
 (segment (start 134.675 96.5) (end 127 96.5) (width 0.2) (layer "B.Cu") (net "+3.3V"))
 (segment (start 126.665 96.835) (end 126.665 98.225) (width 0.2) (layer "B.Cu") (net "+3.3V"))
 (segment (start 127 96.5) (end 126.665 96.835) (width 0.2) (layer "B.Cu") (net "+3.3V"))
 (segment (start 150.612648 84.825) (end 150.9 85.112352) (width 0.2) (layer "F.Cu") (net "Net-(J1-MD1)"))
 (segment (start 148.65 85.5) (end 149.325 84.825) (width 0.2) (layer "F.Cu") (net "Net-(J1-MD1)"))
 (segment (start 150.9 88.77) (end 148.47 91.2) (width 0.2) (layer "F.Cu") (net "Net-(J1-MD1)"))
 (segment (start 149.325 84.825) (end 150.612648 84.825) (width 0.2) (layer "F.Cu") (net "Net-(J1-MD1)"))
 (segment (start 150.9 85.112352) (end 150.9 88.77) (width 0.2) (layer "F.Cu") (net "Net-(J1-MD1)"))
 (segment (start 147.08 92.35) (end 145.93 91.2) (width 0.2) (layer "F.Cu") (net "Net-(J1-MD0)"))
 (segment (start 151.85 85.6) (end 151.85 89.446346) (width 0.2) (layer "F.Cu") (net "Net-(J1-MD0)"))
 (segment (start 151.85 89.446346) (end 148.946346 92.35) (width 0.2) (layer "F.Cu") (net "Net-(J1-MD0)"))
 (segment (start 148.946346 92.35) (end 147.08 92.35) (width 0.2) (layer "F.Cu") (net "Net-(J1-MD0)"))
 (segment (start 141.175 94.325) (end 139.8 95.7) (width 0.2) (layer "F.Cu") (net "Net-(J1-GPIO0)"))
 (segment (start 142.215 93.74) (end 145.93 93.74) (width 0.2) (layer "F.Cu") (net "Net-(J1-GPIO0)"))
 (segment (start 141.175 92.7) (end 142.215 93.74) (width 0.2) (layer "F.Cu") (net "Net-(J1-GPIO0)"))
 (segment (start 141.175 92.7) (end 141.175 94.325) (width 0.2) (layer "F.Cu") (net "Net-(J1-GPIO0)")))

